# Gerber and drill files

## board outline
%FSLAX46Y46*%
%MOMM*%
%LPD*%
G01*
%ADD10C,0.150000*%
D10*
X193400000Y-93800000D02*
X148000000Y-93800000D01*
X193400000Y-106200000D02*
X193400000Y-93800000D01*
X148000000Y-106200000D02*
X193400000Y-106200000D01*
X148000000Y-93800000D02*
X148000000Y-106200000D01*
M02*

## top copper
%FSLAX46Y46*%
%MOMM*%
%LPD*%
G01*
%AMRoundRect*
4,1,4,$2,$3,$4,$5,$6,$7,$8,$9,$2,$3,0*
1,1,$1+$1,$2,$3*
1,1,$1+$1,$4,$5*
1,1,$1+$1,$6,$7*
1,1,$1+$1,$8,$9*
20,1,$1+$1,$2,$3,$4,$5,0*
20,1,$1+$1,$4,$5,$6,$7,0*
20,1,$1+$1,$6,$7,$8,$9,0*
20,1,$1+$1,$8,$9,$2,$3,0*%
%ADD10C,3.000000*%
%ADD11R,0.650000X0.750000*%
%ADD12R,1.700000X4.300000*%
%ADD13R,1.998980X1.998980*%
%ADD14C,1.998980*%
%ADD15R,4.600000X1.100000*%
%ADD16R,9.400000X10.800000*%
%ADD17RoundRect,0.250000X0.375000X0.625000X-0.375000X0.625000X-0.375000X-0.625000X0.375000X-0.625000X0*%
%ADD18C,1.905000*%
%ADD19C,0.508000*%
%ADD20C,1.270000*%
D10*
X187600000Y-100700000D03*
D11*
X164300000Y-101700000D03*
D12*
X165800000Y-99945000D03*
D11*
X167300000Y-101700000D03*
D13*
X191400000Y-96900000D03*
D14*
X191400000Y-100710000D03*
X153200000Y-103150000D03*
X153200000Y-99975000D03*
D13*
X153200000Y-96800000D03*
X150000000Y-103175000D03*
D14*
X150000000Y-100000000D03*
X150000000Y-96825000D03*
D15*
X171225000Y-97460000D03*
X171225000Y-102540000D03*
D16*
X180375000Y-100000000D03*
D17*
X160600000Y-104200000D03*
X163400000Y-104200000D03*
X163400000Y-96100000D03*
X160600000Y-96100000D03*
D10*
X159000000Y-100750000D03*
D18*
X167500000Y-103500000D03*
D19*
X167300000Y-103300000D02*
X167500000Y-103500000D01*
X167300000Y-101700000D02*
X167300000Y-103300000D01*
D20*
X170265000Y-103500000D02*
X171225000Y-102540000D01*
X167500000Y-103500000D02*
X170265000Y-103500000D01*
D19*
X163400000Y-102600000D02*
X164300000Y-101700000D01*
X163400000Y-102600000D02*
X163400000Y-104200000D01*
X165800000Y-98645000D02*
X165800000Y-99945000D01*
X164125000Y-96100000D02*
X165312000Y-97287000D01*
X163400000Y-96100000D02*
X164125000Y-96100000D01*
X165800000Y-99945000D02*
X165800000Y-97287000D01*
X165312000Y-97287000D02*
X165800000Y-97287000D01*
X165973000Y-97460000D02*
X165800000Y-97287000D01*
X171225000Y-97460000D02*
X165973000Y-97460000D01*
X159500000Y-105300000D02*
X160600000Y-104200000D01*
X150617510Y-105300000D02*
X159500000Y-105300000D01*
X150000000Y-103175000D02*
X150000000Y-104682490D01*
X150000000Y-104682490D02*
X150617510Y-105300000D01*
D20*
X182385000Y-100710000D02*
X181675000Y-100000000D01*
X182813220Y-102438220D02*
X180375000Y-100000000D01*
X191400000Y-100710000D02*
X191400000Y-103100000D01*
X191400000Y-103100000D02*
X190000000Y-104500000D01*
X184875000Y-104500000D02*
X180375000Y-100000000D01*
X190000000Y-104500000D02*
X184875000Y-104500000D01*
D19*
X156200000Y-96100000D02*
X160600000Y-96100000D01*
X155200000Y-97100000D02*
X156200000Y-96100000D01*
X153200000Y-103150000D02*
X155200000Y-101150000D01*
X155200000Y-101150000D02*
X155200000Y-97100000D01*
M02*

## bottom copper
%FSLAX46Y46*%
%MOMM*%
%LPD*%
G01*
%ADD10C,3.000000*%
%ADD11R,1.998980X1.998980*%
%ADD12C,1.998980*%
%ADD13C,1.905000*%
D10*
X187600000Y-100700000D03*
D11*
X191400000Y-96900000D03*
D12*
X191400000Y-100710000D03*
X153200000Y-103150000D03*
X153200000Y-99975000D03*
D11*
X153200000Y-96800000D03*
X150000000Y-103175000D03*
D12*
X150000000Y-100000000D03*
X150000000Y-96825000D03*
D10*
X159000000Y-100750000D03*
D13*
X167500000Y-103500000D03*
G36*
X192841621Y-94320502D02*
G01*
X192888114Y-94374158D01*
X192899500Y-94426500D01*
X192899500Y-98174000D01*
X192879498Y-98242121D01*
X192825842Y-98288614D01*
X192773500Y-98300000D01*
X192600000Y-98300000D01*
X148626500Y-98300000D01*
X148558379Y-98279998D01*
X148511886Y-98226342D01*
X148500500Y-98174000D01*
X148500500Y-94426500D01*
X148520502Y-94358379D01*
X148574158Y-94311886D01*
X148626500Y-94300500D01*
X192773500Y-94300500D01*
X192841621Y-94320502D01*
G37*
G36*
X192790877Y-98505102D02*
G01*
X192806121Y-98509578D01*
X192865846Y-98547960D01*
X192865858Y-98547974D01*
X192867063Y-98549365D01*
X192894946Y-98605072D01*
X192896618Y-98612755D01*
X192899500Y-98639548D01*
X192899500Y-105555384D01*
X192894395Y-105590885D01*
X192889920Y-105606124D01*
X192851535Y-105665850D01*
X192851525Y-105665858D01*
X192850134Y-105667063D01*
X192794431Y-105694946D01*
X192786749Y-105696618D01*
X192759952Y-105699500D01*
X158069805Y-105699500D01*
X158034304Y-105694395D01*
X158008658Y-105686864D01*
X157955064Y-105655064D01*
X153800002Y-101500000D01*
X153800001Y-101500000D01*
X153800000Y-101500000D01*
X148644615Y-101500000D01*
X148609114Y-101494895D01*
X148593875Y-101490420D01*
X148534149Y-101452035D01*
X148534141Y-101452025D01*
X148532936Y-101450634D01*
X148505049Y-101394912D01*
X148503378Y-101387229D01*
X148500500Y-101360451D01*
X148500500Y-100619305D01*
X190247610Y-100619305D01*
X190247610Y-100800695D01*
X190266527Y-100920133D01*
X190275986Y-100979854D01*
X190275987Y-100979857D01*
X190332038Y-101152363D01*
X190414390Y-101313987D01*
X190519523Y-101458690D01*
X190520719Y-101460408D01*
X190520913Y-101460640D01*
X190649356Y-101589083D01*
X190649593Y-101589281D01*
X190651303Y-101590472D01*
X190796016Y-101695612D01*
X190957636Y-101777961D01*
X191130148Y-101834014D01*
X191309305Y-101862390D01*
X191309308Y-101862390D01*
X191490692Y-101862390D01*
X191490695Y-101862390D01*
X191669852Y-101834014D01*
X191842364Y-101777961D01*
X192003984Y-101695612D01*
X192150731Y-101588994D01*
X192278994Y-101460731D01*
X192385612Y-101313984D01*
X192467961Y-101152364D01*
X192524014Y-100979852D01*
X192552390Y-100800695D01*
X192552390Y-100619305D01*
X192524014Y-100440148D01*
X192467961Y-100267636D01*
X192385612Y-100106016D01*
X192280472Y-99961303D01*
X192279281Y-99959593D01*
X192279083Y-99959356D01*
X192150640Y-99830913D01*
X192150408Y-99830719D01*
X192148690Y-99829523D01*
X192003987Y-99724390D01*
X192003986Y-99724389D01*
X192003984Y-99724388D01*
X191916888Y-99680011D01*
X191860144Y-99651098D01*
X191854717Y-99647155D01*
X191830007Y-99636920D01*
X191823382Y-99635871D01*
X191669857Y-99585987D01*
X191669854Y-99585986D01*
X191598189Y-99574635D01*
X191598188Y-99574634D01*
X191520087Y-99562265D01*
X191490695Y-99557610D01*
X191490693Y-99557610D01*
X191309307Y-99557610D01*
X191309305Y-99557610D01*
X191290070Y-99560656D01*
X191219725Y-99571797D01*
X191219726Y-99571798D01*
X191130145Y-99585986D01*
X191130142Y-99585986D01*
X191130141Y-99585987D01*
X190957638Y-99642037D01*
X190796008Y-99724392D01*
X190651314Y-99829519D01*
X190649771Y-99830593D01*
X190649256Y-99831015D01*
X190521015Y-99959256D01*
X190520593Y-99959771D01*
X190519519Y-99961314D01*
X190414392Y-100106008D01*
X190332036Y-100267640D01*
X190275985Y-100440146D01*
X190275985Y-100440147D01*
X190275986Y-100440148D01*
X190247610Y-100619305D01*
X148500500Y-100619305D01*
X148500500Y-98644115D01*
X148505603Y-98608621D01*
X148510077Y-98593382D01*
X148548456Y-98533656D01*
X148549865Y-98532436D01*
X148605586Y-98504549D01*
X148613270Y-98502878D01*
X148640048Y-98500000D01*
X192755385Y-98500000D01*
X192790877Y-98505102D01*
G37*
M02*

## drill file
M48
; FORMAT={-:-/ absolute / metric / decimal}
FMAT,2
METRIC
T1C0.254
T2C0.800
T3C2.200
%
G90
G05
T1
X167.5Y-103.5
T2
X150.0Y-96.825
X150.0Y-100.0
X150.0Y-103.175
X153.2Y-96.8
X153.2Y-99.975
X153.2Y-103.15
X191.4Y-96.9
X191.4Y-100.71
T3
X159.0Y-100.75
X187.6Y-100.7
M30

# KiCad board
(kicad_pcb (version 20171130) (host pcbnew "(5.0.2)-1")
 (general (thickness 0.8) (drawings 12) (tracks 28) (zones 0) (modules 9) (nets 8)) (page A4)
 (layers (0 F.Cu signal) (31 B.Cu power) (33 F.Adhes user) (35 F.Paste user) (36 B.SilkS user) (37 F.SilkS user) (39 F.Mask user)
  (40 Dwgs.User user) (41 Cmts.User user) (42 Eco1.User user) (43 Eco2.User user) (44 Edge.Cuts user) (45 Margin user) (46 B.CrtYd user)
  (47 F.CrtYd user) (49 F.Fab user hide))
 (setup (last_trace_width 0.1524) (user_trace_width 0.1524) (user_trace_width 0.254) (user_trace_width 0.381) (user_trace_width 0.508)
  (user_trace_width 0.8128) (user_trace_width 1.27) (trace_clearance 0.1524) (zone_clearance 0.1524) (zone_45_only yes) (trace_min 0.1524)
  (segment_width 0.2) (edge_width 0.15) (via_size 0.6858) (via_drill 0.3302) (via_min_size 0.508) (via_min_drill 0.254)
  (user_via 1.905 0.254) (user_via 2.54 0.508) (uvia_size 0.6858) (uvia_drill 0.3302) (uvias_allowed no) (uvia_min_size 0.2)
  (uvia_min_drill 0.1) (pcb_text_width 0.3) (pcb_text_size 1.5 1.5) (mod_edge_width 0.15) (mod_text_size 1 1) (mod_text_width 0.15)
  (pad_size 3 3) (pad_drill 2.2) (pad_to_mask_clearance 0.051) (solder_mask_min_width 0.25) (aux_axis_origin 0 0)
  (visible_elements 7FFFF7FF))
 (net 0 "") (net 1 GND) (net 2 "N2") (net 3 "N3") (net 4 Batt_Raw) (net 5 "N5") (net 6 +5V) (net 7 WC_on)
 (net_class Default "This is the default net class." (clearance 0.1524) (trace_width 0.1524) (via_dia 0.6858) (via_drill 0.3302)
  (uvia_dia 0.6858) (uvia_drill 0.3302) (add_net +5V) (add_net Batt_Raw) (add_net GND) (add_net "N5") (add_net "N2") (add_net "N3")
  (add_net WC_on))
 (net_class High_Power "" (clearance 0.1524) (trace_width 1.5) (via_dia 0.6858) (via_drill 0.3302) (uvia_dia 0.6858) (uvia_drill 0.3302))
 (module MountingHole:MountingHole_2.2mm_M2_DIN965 (layer F.Cu) (at 187.6 100.7)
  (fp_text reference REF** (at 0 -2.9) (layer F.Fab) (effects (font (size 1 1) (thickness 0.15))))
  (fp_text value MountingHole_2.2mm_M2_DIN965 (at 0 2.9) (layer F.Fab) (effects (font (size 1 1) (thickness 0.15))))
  (pad "" thru_hole circle (at 0 0) (size 3 3) (drill 2.2) (layers *.Cu *.Mask) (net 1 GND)))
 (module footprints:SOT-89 (layer F.Cu) (at 165.8 101.7)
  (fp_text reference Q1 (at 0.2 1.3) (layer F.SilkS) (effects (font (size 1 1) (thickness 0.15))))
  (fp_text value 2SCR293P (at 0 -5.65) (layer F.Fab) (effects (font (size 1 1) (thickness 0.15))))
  (pad 1 smd rect (at -1.5 0) (size 0.65 0.75) (layers F.Cu F.Paste F.Mask) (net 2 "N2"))
  (pad 2 smd rect (at 0 -1.755) (size 1.7 4.3) (layers F.Cu F.Paste F.Mask) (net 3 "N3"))
  (pad 3 smd rect (at 1.5 0) (size 0.65 0.75) (layers F.Cu F.Paste F.Mask) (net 1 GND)))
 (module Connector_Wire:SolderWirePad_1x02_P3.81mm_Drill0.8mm (layer F.Cu) (at 191.4 96.9 270)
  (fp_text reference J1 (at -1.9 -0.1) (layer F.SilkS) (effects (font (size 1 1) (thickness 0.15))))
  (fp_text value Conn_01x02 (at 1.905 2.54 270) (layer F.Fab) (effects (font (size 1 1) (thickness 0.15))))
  (pad 1 thru_hole rect (at 0 0 270) (size 1.99898 1.99898) (drill 0.8001) (layers *.Cu *.Mask) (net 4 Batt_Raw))
  (pad 2 thru_hole circle (at 3.81 0 270) (size 1.99898 1.99898) (drill 0.8001) (layers *.Cu *.Mask) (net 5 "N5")))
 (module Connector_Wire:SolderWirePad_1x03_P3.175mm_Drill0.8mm (layer F.Cu) (at 153.2 96.8 270)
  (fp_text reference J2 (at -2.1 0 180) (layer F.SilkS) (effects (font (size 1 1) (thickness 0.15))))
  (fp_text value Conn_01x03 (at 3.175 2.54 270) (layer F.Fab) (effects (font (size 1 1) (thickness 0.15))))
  (pad 3 thru_hole circle (at 6.35 0 270) (size 1.99898 1.99898) (drill 0.8001) (layers *.Cu *.Mask) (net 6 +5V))
  (pad 2 thru_hole circle (at 3.175 0 270) (size 1.99898 1.99898) (drill 0.8001) (layers *.Cu *.Mask) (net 1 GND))
  (pad 1 thru_hole rect (at 0 0 270) (size 1.99898 1.99898) (drill 0.8001) (layers *.Cu *.Mask) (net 4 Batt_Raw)))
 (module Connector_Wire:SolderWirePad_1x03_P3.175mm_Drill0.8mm (layer F.Cu) (at 150 103.175 90)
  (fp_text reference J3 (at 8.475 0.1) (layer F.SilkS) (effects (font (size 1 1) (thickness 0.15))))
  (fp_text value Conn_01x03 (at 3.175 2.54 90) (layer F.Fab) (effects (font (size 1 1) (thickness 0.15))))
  (pad 1 thru_hole rect (at 0 0 90) (size 1.99898 1.99898) (drill 0.8001) (layers *.Cu *.Mask) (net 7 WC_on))
  (pad 2 thru_hole circle (at 3.175 0 90) (size 1.99898 1.99898) (drill 0.8001) (layers *.Cu *.Mask) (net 1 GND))
  (pad 3 thru_hole circle (at 6.35 0 90) (size 1.99898 1.99898) (drill 0.8001) (layers *.Cu *.Mask) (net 4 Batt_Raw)))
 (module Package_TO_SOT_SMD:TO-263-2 (layer F.Cu) (at 177 100)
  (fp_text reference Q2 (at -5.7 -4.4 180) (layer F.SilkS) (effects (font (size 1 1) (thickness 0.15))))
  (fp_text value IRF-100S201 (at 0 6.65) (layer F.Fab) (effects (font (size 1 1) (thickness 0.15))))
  (pad 1 smd rect (at -5.775 -2.54) (size 4.6 1.1) (layers F.Cu F.Paste F.Mask) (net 3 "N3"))
  (pad 3 smd rect (at -5.775 2.54) (size 4.6 1.1) (layers F.Cu F.Paste F.Mask) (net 1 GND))
  (pad 2 smd rect (at 3.375 0) (size 9.4 10.8) (layers F.Cu F.Mask) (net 5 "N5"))
  (pad "" smd rect (at 5.8 2.775) (size 4.55 5.25) (layers F.Paste))
  (pad "" smd rect (at 0.95 -2.775) (size 4.55 5.25) (layers F.Paste))
  (pad "" smd rect (at 5.8 -2.775) (size 4.55 5.25) (layers F.Paste))
  (pad "" smd rect (at 0.95 2.775) (size 4.55 5.25) (layers F.Paste)))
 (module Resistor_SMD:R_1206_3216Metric (layer F.Cu) (at 162 104.2 180)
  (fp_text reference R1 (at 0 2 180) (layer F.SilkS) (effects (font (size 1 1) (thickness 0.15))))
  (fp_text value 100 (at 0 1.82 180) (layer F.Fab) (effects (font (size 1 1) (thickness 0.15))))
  (pad 2 smd roundrect (at 1.4 0 180) (size 1.25 1.75) (layers F.Cu F.Paste F.Mask) (roundrect_rratio 0.2) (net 7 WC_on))
  (pad 1 smd roundrect (at -1.4 0 180) (size 1.25 1.75) (layers F.Cu F.Paste F.Mask) (roundrect_rratio 0.2) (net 2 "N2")))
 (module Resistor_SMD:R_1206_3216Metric (layer F.Cu) (at 162 96.1 180)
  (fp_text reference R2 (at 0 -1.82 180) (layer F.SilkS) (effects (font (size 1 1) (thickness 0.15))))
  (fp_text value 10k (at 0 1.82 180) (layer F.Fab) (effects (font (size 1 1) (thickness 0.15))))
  (pad 1 smd roundrect (at -1.4 0 180) (size 1.25 1.75) (layers F.Cu F.Paste F.Mask) (roundrect_rratio 0.2) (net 3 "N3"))
  (pad 2 smd roundrect (at 1.4 0 180) (size 1.25 1.75) (layers F.Cu F.Paste F.Mask) (roundrect_rratio 0.2) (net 6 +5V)))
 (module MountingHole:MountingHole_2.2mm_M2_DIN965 (layer F.Cu) (at 159 100.75)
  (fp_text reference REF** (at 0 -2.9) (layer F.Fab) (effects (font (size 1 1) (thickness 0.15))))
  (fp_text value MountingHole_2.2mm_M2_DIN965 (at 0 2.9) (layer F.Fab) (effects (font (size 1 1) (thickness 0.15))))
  (pad "" thru_hole circle (at 0 0) (size 3 3) (drill 2.2) (layers *.Cu *.Mask) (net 1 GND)))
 (gr_line (start 193.4 93.8) (end 148 93.8) (layer Edge.Cuts) (width 0.15))
 (gr_line (start 193.4 106.2) (end 193.4 93.8) (layer Edge.Cuts) (width 0.15))
 (gr_line (start 148 106.2) (end 193.4 106.2) (layer Edge.Cuts) (width 0.15))
 (gr_line (start 148 93.8) (end 148 106.2) (layer Edge.Cuts) (width 0.15))
 (via (at 167.5 103.5) (size 1.905) (drill 0.254) (layers F.Cu B.Cu) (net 1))
 (segment (start 167.3 103.3) (end 167.5 103.5) (width 0.508) (layer F.Cu) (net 1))
 (segment (start 167.3 101.7) (end 167.3 103.3) (width 0.508) (layer F.Cu) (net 1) (status 10))
 (segment (start 170.265 103.5) (end 171.225 102.54) (width 1.27) (layer F.Cu) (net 1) (status 20))
 (segment (start 167.5 103.5) (end 170.265 103.5) (width 1.27) (layer F.Cu) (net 1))
 (segment (start 163.4 102.6) (end 164.3 101.7) (width 0.508) (layer F.Cu) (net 2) (status 20))
 (segment (start 163.4 102.6) (end 163.4 104.2) (width 0.508) (layer F.Cu) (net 2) (status 20))
 (segment (start 165.8 98.645) (end 165.8 99.945) (width 0.508) (layer F.Cu) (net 3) (status 30))
 (segment (start 164.125 96.1) (end 165.312 97.287) (width 0.508) (layer F.Cu) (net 3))
 (segment (start 163.4 96.1) (end 164.125 96.1) (width 0.508) (layer F.Cu) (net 3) (status 10))
 (segment (start 165.8 99.945) (end 165.8 97.287) (width 0.508) (layer F.Cu) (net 3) (status 10))
 (segment (start 165.312 97.287) (end 165.8 97.287) (width 0.508) (layer F.Cu) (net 3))
 (segment (start 165.973 97.46) (end 165.8 97.287) (width 0.508) (layer F.Cu) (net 3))
 (segment (start 171.225 97.46) (end 165.973 97.46) (width 0.508) (layer F.Cu) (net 3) (status 10))
 (segment (start 159.5 105.3) (end 160.6 104.2) (width 0.508) (layer F.Cu) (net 7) (status 20))
 (segment (start 150.61751 105.3) (end 159.5 105.3) (width 0.508) (layer F.Cu) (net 7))
 (segment (start 150 103.175) (end 150 104.68249) (width 0.508) (layer F.Cu) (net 7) (status 10))
 (segment (start 150 104.68249) (end 150.61751 105.3) (width 0.508) (layer F.Cu) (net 7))
 (segment (start 182.385 100.71) (end 181.675 100) (width 1.27) (layer F.Cu) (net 5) (status 30))
 (segment (start 182.81322 102.43822) (end 180.375 100) (width 1.27) (layer F.Cu) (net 5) (status 30))
 (segment (start 191.4 100.71) (end 191.4 103.1) (width 1.27) (layer F.Cu) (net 5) (status 10))
 (segment (start 191.4 103.1) (end 190 104.5) (width 1.27) (layer F.Cu) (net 5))
 (segment (start 184.875 104.5) (end 180.375 100) (width 1.27) (layer F.Cu) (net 5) (status 30))
 (segment (start 190 104.5) (end 184.875 104.5) (width 1.27) (layer F.Cu) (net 5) (status 20))
 (segment (start 156.2 96.1) (end 160.6 96.1) (width 0.508) (layer F.Cu) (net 6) (status 20))
 (segment (start 155.2 97.1) (end 156.2 96.1) (width 0.508) (layer F.Cu) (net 6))
 (segment (start 153.2 103.15) (end 155.2 101.15) (width 0.508) (layer F.Cu) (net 6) (status 10))
 (segment (start 155.2 101.15) (end 155.2 97.1) (width 0.508) (layer F.Cu) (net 6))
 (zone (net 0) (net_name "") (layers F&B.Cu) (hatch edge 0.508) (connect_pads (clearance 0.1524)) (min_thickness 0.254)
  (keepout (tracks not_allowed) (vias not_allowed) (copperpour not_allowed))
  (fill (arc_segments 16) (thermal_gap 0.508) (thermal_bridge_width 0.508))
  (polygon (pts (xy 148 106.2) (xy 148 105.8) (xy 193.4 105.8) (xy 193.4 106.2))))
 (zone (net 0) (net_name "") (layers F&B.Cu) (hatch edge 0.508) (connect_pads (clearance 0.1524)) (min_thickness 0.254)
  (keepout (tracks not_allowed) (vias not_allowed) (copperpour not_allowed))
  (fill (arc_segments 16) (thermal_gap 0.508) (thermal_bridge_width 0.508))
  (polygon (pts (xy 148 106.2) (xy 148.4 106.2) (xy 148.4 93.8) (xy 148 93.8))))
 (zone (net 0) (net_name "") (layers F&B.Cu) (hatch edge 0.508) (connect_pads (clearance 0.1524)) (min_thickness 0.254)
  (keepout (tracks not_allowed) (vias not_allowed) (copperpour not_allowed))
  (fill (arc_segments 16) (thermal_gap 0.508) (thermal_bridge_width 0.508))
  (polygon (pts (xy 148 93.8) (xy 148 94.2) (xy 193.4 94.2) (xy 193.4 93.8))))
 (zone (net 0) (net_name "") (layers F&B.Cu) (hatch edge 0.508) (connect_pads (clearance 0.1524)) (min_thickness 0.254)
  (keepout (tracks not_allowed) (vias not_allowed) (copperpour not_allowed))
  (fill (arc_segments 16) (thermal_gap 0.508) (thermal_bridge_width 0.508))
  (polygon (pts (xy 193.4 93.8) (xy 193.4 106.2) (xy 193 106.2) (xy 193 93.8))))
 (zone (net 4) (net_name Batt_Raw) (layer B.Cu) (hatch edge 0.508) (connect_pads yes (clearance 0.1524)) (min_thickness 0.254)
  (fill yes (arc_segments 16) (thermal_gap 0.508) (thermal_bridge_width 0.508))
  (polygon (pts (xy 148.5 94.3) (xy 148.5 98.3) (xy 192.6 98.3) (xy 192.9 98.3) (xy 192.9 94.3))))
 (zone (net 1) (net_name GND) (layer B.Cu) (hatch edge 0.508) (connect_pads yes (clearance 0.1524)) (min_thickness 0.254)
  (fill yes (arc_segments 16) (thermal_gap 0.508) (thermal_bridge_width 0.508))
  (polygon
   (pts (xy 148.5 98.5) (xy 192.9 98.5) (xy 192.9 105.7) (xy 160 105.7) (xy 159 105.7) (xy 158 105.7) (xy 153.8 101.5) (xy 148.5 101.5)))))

